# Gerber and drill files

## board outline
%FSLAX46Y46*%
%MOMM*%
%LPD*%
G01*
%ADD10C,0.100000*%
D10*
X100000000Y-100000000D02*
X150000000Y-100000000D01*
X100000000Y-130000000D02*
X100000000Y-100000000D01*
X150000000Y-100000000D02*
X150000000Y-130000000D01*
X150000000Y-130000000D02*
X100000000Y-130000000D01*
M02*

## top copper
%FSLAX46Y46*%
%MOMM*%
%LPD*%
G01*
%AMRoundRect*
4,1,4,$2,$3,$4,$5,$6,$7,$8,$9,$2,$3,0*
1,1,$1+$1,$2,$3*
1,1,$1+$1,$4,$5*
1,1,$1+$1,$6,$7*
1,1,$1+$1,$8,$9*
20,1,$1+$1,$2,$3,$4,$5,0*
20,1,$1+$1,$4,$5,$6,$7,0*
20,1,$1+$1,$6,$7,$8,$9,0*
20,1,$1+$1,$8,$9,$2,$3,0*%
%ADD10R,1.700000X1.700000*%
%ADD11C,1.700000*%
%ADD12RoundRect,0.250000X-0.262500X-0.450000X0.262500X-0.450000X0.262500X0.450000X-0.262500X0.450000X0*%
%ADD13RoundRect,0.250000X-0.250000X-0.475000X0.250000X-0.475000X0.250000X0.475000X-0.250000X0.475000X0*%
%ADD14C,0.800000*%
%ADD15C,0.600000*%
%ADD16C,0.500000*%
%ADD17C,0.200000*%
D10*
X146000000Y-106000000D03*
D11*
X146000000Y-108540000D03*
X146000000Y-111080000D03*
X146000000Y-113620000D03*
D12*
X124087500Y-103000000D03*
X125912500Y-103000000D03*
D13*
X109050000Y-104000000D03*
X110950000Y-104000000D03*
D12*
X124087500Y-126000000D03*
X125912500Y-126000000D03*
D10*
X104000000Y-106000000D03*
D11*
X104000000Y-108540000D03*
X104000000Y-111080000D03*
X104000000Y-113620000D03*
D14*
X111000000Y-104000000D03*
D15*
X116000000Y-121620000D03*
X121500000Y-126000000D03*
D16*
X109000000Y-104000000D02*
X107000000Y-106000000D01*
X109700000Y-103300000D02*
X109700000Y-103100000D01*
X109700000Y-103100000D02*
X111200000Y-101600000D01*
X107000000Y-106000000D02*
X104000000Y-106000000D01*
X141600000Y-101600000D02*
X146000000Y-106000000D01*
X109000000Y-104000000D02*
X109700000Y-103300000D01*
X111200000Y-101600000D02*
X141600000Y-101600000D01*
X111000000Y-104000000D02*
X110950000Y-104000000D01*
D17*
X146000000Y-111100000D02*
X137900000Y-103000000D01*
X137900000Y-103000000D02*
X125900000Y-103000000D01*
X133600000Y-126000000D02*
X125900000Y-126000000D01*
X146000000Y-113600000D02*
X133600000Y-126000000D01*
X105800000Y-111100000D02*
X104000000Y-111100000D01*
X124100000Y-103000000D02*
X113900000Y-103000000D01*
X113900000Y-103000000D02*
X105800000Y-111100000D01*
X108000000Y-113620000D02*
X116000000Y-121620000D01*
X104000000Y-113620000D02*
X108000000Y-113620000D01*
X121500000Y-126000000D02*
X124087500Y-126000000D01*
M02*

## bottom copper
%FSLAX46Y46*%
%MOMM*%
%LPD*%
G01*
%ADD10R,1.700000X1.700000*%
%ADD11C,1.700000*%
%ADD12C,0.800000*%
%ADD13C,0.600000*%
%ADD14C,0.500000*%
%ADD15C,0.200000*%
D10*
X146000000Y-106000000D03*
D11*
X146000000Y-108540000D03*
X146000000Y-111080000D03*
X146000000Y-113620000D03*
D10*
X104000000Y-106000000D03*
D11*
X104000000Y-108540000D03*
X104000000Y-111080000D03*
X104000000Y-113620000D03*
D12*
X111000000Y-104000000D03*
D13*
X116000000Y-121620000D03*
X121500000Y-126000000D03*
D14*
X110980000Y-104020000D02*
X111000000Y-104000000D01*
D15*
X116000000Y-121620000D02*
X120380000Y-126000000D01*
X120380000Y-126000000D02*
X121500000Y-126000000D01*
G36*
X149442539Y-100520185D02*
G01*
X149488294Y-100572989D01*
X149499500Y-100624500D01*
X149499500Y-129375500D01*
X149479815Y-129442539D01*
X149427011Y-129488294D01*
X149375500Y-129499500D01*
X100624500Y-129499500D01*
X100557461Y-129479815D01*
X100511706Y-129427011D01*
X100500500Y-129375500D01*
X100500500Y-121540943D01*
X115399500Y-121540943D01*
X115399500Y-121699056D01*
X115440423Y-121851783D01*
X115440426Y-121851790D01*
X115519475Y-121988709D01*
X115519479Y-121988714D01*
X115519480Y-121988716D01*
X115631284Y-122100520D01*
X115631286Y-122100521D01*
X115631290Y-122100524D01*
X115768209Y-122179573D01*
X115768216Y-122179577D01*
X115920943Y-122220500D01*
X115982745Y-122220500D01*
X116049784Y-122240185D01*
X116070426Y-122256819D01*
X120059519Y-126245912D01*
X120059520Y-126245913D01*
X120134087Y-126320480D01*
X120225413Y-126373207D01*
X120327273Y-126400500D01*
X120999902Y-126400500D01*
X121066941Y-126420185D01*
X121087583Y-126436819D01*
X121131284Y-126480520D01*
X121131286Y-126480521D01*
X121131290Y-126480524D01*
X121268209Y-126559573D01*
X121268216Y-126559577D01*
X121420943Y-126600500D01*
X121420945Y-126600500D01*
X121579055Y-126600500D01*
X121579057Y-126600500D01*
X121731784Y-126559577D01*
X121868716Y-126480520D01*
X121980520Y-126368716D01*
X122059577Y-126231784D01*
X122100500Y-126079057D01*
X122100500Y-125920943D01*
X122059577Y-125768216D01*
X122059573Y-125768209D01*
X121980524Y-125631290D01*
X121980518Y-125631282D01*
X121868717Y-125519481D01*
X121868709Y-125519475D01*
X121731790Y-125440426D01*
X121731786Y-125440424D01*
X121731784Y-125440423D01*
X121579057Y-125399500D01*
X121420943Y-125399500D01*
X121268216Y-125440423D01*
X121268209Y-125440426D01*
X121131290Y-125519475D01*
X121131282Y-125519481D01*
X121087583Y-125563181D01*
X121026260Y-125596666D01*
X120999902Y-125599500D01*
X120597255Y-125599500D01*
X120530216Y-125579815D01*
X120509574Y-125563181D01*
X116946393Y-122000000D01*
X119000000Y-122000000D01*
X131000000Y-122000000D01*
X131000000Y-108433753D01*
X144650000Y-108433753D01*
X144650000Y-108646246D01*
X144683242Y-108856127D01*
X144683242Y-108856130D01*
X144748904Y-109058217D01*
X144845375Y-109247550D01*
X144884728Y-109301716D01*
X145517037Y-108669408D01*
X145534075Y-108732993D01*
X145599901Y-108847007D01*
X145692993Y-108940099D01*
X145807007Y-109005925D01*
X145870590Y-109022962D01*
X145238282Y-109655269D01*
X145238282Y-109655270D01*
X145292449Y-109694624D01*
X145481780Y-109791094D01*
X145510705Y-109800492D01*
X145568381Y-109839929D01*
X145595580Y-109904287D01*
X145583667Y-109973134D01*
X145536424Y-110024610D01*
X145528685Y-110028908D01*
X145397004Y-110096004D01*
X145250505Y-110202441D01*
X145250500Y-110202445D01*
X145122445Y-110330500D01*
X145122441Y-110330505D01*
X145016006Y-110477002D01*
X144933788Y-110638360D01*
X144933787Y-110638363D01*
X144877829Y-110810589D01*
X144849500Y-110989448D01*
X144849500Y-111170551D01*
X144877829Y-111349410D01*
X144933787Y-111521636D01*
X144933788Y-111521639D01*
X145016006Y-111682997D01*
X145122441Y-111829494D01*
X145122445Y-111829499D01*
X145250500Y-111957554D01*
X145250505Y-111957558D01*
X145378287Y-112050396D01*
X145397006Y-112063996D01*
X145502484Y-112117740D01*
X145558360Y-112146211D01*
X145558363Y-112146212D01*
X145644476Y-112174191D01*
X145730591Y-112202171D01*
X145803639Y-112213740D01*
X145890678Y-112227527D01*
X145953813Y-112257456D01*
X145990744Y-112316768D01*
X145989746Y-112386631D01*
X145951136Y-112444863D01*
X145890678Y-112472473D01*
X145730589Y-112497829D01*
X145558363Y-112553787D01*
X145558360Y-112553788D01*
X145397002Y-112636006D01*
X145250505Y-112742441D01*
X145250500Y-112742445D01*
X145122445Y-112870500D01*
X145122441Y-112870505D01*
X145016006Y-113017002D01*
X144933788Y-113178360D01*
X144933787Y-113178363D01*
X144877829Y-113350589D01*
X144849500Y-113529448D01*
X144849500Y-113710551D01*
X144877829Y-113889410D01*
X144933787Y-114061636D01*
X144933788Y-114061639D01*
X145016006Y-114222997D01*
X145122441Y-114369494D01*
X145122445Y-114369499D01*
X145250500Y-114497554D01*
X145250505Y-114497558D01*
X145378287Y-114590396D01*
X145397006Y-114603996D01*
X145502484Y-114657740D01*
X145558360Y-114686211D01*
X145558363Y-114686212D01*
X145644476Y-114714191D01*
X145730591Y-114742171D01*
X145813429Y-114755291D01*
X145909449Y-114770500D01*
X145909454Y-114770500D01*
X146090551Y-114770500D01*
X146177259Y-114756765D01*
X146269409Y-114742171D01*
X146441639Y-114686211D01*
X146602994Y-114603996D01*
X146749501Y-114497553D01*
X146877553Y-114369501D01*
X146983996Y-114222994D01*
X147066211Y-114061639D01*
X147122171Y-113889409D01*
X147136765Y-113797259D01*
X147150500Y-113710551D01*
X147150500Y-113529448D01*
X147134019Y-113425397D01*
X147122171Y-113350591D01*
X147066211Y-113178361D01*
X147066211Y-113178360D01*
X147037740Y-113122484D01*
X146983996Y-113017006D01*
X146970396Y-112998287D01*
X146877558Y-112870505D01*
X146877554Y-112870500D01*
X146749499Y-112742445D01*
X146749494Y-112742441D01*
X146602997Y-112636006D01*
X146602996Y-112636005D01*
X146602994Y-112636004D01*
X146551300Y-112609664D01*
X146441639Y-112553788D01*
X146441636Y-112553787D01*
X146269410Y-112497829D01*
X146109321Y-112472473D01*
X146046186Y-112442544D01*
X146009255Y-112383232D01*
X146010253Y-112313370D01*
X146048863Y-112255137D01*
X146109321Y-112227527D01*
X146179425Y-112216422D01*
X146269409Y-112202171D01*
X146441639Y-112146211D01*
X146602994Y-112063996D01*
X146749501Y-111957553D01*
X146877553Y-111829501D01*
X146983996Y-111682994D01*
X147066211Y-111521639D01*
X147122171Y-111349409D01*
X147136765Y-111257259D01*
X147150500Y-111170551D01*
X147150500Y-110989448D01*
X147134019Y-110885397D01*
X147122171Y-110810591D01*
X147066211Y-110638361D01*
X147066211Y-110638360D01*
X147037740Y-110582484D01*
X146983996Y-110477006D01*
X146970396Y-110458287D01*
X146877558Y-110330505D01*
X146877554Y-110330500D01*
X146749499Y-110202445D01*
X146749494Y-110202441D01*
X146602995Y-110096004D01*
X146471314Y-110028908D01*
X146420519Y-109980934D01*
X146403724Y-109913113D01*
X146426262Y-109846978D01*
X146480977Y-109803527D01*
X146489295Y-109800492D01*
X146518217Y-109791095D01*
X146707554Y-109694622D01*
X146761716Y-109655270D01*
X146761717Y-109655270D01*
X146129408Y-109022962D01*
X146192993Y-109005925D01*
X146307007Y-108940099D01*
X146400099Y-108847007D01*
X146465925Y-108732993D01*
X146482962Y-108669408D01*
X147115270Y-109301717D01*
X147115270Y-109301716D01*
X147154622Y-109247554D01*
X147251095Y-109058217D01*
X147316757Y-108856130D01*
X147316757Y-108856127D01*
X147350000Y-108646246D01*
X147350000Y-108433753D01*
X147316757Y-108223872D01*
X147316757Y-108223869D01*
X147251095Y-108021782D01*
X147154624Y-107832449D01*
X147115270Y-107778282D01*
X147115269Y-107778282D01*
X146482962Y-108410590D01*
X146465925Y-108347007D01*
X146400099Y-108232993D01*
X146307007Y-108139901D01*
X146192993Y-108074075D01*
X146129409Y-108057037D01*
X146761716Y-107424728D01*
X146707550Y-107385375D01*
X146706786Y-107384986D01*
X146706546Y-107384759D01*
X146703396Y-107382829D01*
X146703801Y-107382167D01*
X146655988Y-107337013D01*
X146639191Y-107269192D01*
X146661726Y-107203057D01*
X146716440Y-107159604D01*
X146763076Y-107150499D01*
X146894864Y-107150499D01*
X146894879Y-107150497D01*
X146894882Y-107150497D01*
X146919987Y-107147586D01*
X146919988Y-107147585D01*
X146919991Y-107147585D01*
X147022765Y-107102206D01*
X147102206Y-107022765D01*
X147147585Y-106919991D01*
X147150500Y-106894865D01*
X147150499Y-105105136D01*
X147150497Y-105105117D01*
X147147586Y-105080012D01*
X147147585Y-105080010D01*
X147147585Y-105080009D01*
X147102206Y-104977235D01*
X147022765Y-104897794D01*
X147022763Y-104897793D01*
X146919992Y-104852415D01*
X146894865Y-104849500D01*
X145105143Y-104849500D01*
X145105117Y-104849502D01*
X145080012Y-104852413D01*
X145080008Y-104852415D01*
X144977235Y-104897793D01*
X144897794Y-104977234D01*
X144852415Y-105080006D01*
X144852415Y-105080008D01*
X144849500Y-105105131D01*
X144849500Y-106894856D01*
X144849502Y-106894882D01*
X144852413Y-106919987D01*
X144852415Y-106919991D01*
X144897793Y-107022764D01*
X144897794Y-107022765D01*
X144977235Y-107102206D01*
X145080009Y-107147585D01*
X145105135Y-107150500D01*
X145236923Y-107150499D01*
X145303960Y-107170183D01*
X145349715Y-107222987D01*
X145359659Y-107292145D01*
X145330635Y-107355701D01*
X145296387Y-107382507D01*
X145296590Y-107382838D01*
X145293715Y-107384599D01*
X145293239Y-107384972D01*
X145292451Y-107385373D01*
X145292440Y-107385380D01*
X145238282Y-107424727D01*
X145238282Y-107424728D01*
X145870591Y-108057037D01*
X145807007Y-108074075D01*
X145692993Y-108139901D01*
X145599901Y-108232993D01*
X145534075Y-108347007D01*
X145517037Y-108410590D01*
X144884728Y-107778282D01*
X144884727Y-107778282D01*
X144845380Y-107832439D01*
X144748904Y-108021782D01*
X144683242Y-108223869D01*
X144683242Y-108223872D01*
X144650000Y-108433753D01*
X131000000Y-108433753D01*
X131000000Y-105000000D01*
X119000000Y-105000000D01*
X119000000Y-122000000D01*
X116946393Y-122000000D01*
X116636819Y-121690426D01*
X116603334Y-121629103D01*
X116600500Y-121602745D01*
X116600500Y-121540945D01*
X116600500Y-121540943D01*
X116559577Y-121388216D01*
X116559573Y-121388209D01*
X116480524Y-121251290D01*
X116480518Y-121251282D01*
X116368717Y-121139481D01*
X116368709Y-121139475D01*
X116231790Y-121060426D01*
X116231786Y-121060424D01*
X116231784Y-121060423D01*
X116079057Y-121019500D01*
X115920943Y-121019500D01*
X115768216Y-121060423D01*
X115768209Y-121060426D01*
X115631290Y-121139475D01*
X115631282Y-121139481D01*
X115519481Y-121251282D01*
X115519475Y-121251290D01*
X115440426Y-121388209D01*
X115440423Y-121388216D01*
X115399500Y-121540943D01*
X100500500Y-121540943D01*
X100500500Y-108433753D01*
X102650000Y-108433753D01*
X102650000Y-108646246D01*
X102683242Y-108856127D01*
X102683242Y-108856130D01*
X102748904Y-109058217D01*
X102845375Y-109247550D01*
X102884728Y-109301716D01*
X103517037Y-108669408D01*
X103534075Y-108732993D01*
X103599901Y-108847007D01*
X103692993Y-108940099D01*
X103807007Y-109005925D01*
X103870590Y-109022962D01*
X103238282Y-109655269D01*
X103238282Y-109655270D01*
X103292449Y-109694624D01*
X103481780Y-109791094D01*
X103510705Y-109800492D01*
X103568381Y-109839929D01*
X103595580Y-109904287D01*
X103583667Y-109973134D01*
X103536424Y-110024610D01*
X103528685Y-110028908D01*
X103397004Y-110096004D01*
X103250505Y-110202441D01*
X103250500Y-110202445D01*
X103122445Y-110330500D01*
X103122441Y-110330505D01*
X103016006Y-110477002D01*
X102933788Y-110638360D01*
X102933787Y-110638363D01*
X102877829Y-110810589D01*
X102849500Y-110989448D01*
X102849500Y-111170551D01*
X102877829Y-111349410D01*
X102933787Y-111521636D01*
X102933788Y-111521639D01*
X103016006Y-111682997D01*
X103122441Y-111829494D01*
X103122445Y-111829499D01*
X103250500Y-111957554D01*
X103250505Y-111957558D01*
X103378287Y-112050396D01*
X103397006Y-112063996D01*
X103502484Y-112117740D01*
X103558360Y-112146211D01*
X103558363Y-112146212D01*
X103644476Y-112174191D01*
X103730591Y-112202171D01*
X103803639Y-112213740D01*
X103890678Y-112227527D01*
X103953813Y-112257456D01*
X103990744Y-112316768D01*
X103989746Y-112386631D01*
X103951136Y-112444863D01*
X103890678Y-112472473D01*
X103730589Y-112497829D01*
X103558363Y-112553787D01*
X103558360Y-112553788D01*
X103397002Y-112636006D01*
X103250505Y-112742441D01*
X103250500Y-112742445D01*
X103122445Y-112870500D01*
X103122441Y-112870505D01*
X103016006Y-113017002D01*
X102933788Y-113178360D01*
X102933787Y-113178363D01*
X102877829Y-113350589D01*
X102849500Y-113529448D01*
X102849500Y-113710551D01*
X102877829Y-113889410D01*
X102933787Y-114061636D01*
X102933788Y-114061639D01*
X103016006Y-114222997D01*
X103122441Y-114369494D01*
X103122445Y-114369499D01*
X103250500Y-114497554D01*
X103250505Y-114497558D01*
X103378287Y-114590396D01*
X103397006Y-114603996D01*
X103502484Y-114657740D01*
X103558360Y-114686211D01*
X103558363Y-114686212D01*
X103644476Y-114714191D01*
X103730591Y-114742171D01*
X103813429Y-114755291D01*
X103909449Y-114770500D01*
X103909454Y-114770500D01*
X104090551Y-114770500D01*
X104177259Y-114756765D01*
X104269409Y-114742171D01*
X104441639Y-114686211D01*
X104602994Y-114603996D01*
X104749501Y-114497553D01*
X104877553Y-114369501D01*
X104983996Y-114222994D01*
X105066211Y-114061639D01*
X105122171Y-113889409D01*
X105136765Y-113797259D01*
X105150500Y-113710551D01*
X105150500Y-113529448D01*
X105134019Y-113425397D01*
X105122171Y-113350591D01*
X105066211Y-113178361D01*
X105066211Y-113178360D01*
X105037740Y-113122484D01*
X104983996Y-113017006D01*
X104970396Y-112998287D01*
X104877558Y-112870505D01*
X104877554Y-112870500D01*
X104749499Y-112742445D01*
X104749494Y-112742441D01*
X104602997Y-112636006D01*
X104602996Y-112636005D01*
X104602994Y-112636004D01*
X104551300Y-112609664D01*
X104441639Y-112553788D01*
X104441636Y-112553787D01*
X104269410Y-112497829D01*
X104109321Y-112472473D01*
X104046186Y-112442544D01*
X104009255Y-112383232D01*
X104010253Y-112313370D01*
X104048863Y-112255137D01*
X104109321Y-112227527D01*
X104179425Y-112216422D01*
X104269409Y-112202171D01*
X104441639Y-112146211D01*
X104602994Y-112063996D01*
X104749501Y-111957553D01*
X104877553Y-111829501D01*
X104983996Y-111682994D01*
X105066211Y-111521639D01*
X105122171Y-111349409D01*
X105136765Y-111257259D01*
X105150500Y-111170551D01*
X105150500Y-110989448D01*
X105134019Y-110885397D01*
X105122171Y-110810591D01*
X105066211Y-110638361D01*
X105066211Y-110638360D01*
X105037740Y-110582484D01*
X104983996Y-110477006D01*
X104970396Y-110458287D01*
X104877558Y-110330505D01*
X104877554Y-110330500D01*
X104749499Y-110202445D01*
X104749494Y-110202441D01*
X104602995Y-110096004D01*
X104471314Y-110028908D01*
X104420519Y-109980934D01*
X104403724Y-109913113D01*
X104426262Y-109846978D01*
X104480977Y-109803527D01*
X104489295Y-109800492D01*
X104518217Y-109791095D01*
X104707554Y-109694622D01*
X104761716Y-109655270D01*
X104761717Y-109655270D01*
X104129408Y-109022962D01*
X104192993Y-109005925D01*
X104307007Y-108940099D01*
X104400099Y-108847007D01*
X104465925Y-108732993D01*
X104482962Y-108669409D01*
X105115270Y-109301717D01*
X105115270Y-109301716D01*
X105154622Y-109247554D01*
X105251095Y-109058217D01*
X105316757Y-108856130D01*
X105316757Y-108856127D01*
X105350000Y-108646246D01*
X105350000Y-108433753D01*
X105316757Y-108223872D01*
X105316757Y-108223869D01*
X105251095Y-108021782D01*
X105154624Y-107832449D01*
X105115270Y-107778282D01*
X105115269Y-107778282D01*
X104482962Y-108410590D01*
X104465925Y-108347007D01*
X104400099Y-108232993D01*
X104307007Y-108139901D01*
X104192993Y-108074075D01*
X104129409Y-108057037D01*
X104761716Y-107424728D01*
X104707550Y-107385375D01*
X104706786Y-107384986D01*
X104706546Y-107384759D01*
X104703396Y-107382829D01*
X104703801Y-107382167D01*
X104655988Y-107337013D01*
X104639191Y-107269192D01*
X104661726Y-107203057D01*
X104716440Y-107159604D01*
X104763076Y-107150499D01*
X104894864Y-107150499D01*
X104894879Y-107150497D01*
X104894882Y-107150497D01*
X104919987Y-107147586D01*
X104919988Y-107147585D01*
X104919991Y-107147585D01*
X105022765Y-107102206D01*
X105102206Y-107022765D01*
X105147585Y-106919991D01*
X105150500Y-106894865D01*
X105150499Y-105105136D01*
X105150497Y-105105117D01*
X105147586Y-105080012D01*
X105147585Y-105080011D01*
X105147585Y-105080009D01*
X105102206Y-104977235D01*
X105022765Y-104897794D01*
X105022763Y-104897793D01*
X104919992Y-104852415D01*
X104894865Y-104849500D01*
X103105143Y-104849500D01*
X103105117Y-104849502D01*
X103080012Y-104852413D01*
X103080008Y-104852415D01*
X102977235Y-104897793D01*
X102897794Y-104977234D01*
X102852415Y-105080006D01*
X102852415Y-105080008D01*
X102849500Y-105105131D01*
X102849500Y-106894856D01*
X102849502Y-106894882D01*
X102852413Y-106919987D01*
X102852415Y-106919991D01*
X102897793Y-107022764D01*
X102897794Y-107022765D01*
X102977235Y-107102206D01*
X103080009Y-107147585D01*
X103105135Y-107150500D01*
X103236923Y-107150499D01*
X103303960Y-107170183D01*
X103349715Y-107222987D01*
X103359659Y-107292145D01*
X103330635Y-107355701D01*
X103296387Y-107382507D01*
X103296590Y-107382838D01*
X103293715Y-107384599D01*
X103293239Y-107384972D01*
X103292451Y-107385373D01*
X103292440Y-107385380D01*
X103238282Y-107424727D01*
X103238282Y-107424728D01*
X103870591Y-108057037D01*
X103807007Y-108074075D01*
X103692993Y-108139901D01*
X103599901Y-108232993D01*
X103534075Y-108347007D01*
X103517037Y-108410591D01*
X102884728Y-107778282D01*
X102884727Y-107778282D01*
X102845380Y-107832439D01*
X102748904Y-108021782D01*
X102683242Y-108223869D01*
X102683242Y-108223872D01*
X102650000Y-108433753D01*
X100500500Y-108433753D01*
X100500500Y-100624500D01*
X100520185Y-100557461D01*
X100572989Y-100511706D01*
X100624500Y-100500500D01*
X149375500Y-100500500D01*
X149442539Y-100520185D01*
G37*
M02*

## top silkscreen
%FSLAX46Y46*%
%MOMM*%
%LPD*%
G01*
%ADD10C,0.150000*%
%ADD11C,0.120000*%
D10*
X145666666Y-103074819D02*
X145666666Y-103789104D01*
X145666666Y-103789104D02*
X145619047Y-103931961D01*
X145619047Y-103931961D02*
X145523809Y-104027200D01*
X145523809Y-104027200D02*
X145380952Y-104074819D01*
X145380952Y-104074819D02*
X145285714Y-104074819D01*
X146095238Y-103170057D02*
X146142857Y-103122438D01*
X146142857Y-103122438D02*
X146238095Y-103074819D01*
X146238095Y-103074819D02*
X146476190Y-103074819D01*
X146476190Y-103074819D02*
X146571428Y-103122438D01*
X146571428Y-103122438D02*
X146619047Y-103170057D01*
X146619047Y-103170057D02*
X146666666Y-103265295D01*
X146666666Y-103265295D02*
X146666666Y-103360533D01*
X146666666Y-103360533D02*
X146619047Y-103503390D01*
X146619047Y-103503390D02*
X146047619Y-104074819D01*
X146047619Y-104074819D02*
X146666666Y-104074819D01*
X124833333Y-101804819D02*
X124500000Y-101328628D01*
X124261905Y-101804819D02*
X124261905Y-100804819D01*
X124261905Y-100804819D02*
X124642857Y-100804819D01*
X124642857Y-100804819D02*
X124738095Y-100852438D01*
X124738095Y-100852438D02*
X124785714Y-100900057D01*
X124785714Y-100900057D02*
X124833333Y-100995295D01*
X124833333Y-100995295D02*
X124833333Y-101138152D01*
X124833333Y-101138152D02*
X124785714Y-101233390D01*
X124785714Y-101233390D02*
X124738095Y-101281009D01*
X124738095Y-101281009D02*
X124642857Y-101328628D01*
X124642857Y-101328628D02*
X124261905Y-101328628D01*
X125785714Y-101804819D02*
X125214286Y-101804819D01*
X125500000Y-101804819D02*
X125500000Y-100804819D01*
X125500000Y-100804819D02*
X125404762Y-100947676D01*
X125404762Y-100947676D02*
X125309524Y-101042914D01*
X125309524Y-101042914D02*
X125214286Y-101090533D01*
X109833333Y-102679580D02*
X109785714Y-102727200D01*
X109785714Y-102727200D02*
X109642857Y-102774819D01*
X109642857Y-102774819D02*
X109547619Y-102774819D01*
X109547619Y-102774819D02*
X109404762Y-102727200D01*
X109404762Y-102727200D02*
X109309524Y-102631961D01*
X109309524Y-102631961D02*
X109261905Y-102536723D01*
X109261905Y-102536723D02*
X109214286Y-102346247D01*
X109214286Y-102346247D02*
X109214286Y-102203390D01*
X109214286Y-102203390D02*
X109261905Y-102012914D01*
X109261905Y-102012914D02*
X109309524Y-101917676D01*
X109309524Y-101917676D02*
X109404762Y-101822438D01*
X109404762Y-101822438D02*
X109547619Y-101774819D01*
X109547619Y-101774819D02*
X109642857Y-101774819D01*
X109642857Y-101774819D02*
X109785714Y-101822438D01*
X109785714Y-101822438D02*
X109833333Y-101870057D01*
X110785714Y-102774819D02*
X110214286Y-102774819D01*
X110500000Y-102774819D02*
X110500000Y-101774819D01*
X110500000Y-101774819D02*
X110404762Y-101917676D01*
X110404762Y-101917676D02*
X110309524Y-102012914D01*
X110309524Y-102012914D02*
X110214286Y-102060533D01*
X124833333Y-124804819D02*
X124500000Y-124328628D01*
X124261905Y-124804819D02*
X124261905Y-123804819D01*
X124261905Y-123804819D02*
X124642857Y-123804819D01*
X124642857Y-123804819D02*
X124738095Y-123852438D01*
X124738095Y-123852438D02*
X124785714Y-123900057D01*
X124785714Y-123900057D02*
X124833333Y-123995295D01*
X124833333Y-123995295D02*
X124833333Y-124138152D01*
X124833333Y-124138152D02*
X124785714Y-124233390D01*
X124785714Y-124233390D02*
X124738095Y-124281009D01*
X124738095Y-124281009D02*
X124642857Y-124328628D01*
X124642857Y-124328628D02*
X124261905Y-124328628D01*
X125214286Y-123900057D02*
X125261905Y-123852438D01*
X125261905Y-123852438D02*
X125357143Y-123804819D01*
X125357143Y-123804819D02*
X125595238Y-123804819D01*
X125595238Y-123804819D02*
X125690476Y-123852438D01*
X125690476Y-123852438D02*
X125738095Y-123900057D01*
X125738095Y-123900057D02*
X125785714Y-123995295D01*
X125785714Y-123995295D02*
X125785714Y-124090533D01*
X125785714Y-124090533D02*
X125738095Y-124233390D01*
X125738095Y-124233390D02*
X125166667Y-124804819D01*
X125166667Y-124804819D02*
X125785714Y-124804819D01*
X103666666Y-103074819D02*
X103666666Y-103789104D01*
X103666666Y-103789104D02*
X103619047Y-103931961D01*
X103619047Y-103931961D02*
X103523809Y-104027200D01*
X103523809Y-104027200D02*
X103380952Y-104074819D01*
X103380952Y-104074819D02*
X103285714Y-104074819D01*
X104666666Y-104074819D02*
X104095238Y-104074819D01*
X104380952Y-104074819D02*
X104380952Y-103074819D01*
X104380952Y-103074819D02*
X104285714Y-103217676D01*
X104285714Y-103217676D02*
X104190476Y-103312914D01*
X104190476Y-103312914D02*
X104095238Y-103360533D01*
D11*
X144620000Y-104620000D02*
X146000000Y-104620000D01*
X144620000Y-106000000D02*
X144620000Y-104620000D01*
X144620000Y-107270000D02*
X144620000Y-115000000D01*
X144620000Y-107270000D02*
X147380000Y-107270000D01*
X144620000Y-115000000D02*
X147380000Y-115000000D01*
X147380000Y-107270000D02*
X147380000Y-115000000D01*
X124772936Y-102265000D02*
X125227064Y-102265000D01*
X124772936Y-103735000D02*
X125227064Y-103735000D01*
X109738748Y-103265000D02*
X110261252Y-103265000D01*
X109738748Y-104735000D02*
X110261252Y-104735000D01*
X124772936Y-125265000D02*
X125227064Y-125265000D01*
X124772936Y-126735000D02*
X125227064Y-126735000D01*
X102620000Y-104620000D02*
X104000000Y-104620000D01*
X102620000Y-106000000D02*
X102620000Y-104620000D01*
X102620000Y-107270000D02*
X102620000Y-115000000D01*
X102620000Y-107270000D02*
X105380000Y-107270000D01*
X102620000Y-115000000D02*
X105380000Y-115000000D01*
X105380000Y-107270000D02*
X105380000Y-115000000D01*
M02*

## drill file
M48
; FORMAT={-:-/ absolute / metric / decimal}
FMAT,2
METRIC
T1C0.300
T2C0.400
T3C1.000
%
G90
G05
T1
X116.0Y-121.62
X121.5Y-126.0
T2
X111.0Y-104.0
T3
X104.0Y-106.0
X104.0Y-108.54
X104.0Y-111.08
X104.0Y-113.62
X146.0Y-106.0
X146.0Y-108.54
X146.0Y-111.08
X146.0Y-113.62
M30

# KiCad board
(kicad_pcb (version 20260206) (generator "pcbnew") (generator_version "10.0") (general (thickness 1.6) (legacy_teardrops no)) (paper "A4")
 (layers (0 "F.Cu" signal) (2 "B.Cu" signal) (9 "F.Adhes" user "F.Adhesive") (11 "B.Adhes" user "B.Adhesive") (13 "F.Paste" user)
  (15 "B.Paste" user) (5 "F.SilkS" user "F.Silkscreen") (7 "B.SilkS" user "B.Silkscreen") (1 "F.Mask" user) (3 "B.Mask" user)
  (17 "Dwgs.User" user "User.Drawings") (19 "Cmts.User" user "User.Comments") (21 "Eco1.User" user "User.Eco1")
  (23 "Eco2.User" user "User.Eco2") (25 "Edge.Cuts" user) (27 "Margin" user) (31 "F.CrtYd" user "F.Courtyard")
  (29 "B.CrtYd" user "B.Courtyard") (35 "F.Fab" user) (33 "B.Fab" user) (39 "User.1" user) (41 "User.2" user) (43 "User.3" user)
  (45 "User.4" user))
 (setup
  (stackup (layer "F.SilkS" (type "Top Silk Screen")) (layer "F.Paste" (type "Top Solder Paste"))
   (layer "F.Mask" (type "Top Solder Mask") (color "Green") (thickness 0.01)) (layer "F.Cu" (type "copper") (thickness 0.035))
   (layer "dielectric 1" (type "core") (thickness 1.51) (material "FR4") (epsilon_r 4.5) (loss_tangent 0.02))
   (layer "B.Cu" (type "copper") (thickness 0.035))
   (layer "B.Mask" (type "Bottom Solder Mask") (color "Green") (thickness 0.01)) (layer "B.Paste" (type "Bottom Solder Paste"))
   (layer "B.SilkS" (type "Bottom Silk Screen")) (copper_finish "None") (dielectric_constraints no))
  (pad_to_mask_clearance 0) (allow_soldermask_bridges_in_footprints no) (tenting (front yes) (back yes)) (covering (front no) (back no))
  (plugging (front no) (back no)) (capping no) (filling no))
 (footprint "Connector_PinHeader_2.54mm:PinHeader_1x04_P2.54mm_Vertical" (layer "F.Cu") (at 146 106)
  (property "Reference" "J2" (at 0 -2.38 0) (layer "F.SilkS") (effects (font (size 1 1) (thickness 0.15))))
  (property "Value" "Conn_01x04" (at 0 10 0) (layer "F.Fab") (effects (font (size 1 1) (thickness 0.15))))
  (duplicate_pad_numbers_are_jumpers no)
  (fp_line (start -1.38 -1.38) (end 0 -1.38) (stroke (width 0.12) (type solid)) (layer "F.SilkS"))
  (fp_line (start -1.38 0) (end -1.38 -1.38) (stroke (width 0.12) (type solid)) (layer "F.SilkS"))
  (fp_line (start -1.38 1.27) (end -1.38 9) (stroke (width 0.12) (type solid)) (layer "F.SilkS"))
  (fp_line (start -1.38 1.27) (end 1.38 1.27) (stroke (width 0.12) (type solid)) (layer "F.SilkS"))
  (fp_line (start -1.38 9) (end 1.38 9) (stroke (width 0.12) (type solid)) (layer "F.SilkS"))
  (fp_line (start 1.38 1.27) (end 1.38 9) (stroke (width 0.12) (type solid)) (layer "F.SilkS"))
  (pad "1" thru_hole rect (at 0 0) (size 1.7 1.7) (drill 1) (layers "*.Cu" "*.Mask") (remove_unused_layers no) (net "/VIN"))
  (pad "2" thru_hole circle (at 0 2.54) (size 1.7 1.7) (drill 1) (layers "*.Cu" "*.Mask") (remove_unused_layers no) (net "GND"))
  (pad "3" thru_hole circle (at 0 5.08) (size 1.7 1.7) (drill 1) (layers "*.Cu" "*.Mask") (remove_unused_layers no) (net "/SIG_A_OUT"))
  (pad "4" thru_hole circle (at 0 7.62) (size 1.7 1.7) (drill 1) (layers "*.Cu" "*.Mask") (remove_unused_layers no) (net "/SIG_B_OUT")))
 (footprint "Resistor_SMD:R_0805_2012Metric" (layer "F.Cu") (at 125 103)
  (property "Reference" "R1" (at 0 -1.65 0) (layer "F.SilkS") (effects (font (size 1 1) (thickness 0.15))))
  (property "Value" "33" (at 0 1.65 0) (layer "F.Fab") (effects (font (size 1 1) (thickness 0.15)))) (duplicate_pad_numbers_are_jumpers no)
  (fp_line (start -0.227064 -0.735) (end 0.227064 -0.735) (stroke (width 0.12) (type solid)) (layer "F.SilkS"))
  (fp_line (start -0.227064 0.735) (end 0.227064 0.735) (stroke (width 0.12) (type solid)) (layer "F.SilkS"))
  (pad "1" smd roundrect (at -0.9125 0) (size 1.025 1.4) (layers "F.Cu" "F.Mask" "F.Paste") (roundrect_rratio 0.243902) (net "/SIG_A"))
  (pad "2" smd roundrect (at 0.9125 0) (size 1.025 1.4) (layers "F.Cu" "F.Mask" "F.Paste") (roundrect_rratio 0.243902) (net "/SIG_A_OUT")))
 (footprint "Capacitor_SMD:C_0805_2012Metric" (layer "F.Cu") (at 110 104)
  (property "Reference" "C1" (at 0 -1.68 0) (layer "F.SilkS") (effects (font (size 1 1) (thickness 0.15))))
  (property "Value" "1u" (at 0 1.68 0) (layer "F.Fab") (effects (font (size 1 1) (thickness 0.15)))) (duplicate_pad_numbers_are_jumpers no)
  (fp_line (start -0.261252 -0.735) (end 0.261252 -0.735) (stroke (width 0.12) (type solid)) (layer "F.SilkS"))
  (fp_line (start -0.261252 0.735) (end 0.261252 0.735) (stroke (width 0.12) (type solid)) (layer "F.SilkS"))
  (pad "1" smd roundrect (at -0.95 0) (size 1 1.45) (layers "F.Cu" "F.Mask" "F.Paste") (roundrect_rratio 0.25) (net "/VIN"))
  (pad "2" smd roundrect (at 0.95 0) (size 1 1.45) (layers "F.Cu" "F.Mask" "F.Paste") (roundrect_rratio 0.25) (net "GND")))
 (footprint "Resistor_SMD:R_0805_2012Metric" (layer "F.Cu") (at 125 126)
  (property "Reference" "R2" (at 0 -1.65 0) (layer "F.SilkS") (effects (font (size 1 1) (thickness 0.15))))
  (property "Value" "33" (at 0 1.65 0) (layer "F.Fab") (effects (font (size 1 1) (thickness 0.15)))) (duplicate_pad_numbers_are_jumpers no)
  (fp_line (start -0.227064 -0.735) (end 0.227064 -0.735) (stroke (width 0.12) (type solid)) (layer "F.SilkS"))
  (fp_line (start -0.227064 0.735) (end 0.227064 0.735) (stroke (width 0.12) (type solid)) (layer "F.SilkS"))
  (pad "1" smd roundrect (at -0.9125 0) (size 1.025 1.4) (layers "F.Cu" "F.Mask" "F.Paste") (roundrect_rratio 0.243902) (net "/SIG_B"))
  (pad "2" smd roundrect (at 0.9125 0) (size 1.025 1.4) (layers "F.Cu" "F.Mask" "F.Paste") (roundrect_rratio 0.243902) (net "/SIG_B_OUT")))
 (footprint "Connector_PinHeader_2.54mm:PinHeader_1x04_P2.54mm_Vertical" (layer "F.Cu") (at 104 106)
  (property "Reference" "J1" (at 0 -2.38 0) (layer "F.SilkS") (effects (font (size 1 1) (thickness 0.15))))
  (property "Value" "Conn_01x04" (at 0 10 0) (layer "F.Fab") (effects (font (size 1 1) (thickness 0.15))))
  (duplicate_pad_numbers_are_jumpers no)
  (fp_line (start -1.38 -1.38) (end 0 -1.38) (stroke (width 0.12) (type solid)) (layer "F.SilkS"))
  (fp_line (start -1.38 0) (end -1.38 -1.38) (stroke (width 0.12) (type solid)) (layer "F.SilkS"))
  (fp_line (start -1.38 1.27) (end -1.38 9) (stroke (width 0.12) (type solid)) (layer "F.SilkS"))
  (fp_line (start -1.38 1.27) (end 1.38 1.27) (stroke (width 0.12) (type solid)) (layer "F.SilkS"))
  (fp_line (start -1.38 9) (end 1.38 9) (stroke (width 0.12) (type solid)) (layer "F.SilkS"))
  (fp_line (start 1.38 1.27) (end 1.38 9) (stroke (width 0.12) (type solid)) (layer "F.SilkS"))
  (pad "1" thru_hole rect (at 0 0) (size 1.7 1.7) (drill 1) (layers "*.Cu" "*.Mask") (remove_unused_layers no) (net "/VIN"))
  (pad "2" thru_hole circle (at 0 2.54) (size 1.7 1.7) (drill 1) (layers "*.Cu" "*.Mask") (remove_unused_layers no) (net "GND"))
  (pad "3" thru_hole circle (at 0 5.08) (size 1.7 1.7) (drill 1) (layers "*.Cu" "*.Mask") (remove_unused_layers no) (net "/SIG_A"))
  (pad "4" thru_hole circle (at 0 7.62) (size 1.7 1.7) (drill 1) (layers "*.Cu" "*.Mask") (remove_unused_layers no) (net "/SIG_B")))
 (gr_line (start 100 100) (end 150 100) (stroke (width 0.1) (type default)) (layer "Edge.Cuts"))
 (gr_line (start 100 130) (end 100 100) (stroke (width 0.1) (type default)) (layer "Edge.Cuts"))
 (gr_line (start 150 100) (end 150 130) (stroke (width 0.1) (type default)) (layer "Edge.Cuts"))
 (gr_line (start 150 130) (end 100 130) (stroke (width 0.1) (type default)) (layer "Edge.Cuts"))
 (segment (start 109 104) (end 107 106) (width 0.5) (layer "F.Cu") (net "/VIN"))
 (segment (start 109.7 103.3) (end 109.7 103.1) (width 0.5) (layer "F.Cu") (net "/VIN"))
 (segment (start 109.7 103.1) (end 111.2 101.6) (width 0.5) (layer "F.Cu") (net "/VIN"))
 (segment (start 107 106) (end 104 106) (width 0.5) (layer "F.Cu") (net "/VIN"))
 (segment (start 141.6 101.6) (end 146 106) (width 0.5) (layer "F.Cu") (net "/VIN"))
 (segment (start 109 104) (end 109.7 103.3) (width 0.5) (layer "F.Cu") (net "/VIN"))
 (segment (start 111.2 101.6) (end 141.6 101.6) (width 0.5) (layer "F.Cu") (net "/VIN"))
 (segment (start 111 104) (end 110.95 104) (width 0.5) (layer "F.Cu") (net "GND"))
 (via (at 111 104) (size 0.8) (drill 0.4) (layers "F.Cu" "B.Cu") (capping yes) (filling yes) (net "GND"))
 (segment (start 110.98 104.02) (end 111 104) (width 0.5) (layer "B.Cu") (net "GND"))
 (segment (start 146 111.1) (end 137.9 103) (width 0.2) (layer "F.Cu") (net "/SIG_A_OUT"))
 (segment (start 137.9 103) (end 125.9 103) (width 0.2) (layer "F.Cu") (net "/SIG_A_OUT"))
 (segment (start 133.6 126) (end 125.9 126) (width 0.2) (layer "F.Cu") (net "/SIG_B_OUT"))
 (segment (start 146 113.6) (end 133.6 126) (width 0.2) (layer "F.Cu") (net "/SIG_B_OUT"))
 (segment (start 105.8 111.1) (end 104 111.1) (width 0.2) (layer "F.Cu") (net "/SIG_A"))
 (segment (start 124.1 103) (end 113.9 103) (width 0.2) (layer "F.Cu") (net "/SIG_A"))
 (segment (start 113.9 103) (end 105.8 111.1) (width 0.2) (layer "F.Cu") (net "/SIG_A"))
 (segment (start 108 113.62) (end 116 121.62) (width 0.2) (locked yes) (layer "F.Cu") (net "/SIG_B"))
 (segment (start 104 113.62) (end 108 113.62) (width 0.2) (locked yes) (layer "F.Cu") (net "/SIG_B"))
 (segment (start 121.5 126) (end 124.0875 126) (width 0.2) (locked yes) (layer "F.Cu") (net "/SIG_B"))
 (via (at 116 121.62) (size 0.6) (drill 0.3) (layers "F.Cu" "B.Cu") (locked yes) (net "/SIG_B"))
 (via (at 121.5 126) (size 0.6) (drill 0.3) (layers "F.Cu" "B.Cu") (locked yes) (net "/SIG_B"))
 (segment (start 116 121.62) (end 120.38 126) (width 0.2) (locked yes) (layer "B.Cu") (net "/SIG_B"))
 (segment (start 120.38 126) (end 121.5 126) (width 0.2) (locked yes) (layer "B.Cu") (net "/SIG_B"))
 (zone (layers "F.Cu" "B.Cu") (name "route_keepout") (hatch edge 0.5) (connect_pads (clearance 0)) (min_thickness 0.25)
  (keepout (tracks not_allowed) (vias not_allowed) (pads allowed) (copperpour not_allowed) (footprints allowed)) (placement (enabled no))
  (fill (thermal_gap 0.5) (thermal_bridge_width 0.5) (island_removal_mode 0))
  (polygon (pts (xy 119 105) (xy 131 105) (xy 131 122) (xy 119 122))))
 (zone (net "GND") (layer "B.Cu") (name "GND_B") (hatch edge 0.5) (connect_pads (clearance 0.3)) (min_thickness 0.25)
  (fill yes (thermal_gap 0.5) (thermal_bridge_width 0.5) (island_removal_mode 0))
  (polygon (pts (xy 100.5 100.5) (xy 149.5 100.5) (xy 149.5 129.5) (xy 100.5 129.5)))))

